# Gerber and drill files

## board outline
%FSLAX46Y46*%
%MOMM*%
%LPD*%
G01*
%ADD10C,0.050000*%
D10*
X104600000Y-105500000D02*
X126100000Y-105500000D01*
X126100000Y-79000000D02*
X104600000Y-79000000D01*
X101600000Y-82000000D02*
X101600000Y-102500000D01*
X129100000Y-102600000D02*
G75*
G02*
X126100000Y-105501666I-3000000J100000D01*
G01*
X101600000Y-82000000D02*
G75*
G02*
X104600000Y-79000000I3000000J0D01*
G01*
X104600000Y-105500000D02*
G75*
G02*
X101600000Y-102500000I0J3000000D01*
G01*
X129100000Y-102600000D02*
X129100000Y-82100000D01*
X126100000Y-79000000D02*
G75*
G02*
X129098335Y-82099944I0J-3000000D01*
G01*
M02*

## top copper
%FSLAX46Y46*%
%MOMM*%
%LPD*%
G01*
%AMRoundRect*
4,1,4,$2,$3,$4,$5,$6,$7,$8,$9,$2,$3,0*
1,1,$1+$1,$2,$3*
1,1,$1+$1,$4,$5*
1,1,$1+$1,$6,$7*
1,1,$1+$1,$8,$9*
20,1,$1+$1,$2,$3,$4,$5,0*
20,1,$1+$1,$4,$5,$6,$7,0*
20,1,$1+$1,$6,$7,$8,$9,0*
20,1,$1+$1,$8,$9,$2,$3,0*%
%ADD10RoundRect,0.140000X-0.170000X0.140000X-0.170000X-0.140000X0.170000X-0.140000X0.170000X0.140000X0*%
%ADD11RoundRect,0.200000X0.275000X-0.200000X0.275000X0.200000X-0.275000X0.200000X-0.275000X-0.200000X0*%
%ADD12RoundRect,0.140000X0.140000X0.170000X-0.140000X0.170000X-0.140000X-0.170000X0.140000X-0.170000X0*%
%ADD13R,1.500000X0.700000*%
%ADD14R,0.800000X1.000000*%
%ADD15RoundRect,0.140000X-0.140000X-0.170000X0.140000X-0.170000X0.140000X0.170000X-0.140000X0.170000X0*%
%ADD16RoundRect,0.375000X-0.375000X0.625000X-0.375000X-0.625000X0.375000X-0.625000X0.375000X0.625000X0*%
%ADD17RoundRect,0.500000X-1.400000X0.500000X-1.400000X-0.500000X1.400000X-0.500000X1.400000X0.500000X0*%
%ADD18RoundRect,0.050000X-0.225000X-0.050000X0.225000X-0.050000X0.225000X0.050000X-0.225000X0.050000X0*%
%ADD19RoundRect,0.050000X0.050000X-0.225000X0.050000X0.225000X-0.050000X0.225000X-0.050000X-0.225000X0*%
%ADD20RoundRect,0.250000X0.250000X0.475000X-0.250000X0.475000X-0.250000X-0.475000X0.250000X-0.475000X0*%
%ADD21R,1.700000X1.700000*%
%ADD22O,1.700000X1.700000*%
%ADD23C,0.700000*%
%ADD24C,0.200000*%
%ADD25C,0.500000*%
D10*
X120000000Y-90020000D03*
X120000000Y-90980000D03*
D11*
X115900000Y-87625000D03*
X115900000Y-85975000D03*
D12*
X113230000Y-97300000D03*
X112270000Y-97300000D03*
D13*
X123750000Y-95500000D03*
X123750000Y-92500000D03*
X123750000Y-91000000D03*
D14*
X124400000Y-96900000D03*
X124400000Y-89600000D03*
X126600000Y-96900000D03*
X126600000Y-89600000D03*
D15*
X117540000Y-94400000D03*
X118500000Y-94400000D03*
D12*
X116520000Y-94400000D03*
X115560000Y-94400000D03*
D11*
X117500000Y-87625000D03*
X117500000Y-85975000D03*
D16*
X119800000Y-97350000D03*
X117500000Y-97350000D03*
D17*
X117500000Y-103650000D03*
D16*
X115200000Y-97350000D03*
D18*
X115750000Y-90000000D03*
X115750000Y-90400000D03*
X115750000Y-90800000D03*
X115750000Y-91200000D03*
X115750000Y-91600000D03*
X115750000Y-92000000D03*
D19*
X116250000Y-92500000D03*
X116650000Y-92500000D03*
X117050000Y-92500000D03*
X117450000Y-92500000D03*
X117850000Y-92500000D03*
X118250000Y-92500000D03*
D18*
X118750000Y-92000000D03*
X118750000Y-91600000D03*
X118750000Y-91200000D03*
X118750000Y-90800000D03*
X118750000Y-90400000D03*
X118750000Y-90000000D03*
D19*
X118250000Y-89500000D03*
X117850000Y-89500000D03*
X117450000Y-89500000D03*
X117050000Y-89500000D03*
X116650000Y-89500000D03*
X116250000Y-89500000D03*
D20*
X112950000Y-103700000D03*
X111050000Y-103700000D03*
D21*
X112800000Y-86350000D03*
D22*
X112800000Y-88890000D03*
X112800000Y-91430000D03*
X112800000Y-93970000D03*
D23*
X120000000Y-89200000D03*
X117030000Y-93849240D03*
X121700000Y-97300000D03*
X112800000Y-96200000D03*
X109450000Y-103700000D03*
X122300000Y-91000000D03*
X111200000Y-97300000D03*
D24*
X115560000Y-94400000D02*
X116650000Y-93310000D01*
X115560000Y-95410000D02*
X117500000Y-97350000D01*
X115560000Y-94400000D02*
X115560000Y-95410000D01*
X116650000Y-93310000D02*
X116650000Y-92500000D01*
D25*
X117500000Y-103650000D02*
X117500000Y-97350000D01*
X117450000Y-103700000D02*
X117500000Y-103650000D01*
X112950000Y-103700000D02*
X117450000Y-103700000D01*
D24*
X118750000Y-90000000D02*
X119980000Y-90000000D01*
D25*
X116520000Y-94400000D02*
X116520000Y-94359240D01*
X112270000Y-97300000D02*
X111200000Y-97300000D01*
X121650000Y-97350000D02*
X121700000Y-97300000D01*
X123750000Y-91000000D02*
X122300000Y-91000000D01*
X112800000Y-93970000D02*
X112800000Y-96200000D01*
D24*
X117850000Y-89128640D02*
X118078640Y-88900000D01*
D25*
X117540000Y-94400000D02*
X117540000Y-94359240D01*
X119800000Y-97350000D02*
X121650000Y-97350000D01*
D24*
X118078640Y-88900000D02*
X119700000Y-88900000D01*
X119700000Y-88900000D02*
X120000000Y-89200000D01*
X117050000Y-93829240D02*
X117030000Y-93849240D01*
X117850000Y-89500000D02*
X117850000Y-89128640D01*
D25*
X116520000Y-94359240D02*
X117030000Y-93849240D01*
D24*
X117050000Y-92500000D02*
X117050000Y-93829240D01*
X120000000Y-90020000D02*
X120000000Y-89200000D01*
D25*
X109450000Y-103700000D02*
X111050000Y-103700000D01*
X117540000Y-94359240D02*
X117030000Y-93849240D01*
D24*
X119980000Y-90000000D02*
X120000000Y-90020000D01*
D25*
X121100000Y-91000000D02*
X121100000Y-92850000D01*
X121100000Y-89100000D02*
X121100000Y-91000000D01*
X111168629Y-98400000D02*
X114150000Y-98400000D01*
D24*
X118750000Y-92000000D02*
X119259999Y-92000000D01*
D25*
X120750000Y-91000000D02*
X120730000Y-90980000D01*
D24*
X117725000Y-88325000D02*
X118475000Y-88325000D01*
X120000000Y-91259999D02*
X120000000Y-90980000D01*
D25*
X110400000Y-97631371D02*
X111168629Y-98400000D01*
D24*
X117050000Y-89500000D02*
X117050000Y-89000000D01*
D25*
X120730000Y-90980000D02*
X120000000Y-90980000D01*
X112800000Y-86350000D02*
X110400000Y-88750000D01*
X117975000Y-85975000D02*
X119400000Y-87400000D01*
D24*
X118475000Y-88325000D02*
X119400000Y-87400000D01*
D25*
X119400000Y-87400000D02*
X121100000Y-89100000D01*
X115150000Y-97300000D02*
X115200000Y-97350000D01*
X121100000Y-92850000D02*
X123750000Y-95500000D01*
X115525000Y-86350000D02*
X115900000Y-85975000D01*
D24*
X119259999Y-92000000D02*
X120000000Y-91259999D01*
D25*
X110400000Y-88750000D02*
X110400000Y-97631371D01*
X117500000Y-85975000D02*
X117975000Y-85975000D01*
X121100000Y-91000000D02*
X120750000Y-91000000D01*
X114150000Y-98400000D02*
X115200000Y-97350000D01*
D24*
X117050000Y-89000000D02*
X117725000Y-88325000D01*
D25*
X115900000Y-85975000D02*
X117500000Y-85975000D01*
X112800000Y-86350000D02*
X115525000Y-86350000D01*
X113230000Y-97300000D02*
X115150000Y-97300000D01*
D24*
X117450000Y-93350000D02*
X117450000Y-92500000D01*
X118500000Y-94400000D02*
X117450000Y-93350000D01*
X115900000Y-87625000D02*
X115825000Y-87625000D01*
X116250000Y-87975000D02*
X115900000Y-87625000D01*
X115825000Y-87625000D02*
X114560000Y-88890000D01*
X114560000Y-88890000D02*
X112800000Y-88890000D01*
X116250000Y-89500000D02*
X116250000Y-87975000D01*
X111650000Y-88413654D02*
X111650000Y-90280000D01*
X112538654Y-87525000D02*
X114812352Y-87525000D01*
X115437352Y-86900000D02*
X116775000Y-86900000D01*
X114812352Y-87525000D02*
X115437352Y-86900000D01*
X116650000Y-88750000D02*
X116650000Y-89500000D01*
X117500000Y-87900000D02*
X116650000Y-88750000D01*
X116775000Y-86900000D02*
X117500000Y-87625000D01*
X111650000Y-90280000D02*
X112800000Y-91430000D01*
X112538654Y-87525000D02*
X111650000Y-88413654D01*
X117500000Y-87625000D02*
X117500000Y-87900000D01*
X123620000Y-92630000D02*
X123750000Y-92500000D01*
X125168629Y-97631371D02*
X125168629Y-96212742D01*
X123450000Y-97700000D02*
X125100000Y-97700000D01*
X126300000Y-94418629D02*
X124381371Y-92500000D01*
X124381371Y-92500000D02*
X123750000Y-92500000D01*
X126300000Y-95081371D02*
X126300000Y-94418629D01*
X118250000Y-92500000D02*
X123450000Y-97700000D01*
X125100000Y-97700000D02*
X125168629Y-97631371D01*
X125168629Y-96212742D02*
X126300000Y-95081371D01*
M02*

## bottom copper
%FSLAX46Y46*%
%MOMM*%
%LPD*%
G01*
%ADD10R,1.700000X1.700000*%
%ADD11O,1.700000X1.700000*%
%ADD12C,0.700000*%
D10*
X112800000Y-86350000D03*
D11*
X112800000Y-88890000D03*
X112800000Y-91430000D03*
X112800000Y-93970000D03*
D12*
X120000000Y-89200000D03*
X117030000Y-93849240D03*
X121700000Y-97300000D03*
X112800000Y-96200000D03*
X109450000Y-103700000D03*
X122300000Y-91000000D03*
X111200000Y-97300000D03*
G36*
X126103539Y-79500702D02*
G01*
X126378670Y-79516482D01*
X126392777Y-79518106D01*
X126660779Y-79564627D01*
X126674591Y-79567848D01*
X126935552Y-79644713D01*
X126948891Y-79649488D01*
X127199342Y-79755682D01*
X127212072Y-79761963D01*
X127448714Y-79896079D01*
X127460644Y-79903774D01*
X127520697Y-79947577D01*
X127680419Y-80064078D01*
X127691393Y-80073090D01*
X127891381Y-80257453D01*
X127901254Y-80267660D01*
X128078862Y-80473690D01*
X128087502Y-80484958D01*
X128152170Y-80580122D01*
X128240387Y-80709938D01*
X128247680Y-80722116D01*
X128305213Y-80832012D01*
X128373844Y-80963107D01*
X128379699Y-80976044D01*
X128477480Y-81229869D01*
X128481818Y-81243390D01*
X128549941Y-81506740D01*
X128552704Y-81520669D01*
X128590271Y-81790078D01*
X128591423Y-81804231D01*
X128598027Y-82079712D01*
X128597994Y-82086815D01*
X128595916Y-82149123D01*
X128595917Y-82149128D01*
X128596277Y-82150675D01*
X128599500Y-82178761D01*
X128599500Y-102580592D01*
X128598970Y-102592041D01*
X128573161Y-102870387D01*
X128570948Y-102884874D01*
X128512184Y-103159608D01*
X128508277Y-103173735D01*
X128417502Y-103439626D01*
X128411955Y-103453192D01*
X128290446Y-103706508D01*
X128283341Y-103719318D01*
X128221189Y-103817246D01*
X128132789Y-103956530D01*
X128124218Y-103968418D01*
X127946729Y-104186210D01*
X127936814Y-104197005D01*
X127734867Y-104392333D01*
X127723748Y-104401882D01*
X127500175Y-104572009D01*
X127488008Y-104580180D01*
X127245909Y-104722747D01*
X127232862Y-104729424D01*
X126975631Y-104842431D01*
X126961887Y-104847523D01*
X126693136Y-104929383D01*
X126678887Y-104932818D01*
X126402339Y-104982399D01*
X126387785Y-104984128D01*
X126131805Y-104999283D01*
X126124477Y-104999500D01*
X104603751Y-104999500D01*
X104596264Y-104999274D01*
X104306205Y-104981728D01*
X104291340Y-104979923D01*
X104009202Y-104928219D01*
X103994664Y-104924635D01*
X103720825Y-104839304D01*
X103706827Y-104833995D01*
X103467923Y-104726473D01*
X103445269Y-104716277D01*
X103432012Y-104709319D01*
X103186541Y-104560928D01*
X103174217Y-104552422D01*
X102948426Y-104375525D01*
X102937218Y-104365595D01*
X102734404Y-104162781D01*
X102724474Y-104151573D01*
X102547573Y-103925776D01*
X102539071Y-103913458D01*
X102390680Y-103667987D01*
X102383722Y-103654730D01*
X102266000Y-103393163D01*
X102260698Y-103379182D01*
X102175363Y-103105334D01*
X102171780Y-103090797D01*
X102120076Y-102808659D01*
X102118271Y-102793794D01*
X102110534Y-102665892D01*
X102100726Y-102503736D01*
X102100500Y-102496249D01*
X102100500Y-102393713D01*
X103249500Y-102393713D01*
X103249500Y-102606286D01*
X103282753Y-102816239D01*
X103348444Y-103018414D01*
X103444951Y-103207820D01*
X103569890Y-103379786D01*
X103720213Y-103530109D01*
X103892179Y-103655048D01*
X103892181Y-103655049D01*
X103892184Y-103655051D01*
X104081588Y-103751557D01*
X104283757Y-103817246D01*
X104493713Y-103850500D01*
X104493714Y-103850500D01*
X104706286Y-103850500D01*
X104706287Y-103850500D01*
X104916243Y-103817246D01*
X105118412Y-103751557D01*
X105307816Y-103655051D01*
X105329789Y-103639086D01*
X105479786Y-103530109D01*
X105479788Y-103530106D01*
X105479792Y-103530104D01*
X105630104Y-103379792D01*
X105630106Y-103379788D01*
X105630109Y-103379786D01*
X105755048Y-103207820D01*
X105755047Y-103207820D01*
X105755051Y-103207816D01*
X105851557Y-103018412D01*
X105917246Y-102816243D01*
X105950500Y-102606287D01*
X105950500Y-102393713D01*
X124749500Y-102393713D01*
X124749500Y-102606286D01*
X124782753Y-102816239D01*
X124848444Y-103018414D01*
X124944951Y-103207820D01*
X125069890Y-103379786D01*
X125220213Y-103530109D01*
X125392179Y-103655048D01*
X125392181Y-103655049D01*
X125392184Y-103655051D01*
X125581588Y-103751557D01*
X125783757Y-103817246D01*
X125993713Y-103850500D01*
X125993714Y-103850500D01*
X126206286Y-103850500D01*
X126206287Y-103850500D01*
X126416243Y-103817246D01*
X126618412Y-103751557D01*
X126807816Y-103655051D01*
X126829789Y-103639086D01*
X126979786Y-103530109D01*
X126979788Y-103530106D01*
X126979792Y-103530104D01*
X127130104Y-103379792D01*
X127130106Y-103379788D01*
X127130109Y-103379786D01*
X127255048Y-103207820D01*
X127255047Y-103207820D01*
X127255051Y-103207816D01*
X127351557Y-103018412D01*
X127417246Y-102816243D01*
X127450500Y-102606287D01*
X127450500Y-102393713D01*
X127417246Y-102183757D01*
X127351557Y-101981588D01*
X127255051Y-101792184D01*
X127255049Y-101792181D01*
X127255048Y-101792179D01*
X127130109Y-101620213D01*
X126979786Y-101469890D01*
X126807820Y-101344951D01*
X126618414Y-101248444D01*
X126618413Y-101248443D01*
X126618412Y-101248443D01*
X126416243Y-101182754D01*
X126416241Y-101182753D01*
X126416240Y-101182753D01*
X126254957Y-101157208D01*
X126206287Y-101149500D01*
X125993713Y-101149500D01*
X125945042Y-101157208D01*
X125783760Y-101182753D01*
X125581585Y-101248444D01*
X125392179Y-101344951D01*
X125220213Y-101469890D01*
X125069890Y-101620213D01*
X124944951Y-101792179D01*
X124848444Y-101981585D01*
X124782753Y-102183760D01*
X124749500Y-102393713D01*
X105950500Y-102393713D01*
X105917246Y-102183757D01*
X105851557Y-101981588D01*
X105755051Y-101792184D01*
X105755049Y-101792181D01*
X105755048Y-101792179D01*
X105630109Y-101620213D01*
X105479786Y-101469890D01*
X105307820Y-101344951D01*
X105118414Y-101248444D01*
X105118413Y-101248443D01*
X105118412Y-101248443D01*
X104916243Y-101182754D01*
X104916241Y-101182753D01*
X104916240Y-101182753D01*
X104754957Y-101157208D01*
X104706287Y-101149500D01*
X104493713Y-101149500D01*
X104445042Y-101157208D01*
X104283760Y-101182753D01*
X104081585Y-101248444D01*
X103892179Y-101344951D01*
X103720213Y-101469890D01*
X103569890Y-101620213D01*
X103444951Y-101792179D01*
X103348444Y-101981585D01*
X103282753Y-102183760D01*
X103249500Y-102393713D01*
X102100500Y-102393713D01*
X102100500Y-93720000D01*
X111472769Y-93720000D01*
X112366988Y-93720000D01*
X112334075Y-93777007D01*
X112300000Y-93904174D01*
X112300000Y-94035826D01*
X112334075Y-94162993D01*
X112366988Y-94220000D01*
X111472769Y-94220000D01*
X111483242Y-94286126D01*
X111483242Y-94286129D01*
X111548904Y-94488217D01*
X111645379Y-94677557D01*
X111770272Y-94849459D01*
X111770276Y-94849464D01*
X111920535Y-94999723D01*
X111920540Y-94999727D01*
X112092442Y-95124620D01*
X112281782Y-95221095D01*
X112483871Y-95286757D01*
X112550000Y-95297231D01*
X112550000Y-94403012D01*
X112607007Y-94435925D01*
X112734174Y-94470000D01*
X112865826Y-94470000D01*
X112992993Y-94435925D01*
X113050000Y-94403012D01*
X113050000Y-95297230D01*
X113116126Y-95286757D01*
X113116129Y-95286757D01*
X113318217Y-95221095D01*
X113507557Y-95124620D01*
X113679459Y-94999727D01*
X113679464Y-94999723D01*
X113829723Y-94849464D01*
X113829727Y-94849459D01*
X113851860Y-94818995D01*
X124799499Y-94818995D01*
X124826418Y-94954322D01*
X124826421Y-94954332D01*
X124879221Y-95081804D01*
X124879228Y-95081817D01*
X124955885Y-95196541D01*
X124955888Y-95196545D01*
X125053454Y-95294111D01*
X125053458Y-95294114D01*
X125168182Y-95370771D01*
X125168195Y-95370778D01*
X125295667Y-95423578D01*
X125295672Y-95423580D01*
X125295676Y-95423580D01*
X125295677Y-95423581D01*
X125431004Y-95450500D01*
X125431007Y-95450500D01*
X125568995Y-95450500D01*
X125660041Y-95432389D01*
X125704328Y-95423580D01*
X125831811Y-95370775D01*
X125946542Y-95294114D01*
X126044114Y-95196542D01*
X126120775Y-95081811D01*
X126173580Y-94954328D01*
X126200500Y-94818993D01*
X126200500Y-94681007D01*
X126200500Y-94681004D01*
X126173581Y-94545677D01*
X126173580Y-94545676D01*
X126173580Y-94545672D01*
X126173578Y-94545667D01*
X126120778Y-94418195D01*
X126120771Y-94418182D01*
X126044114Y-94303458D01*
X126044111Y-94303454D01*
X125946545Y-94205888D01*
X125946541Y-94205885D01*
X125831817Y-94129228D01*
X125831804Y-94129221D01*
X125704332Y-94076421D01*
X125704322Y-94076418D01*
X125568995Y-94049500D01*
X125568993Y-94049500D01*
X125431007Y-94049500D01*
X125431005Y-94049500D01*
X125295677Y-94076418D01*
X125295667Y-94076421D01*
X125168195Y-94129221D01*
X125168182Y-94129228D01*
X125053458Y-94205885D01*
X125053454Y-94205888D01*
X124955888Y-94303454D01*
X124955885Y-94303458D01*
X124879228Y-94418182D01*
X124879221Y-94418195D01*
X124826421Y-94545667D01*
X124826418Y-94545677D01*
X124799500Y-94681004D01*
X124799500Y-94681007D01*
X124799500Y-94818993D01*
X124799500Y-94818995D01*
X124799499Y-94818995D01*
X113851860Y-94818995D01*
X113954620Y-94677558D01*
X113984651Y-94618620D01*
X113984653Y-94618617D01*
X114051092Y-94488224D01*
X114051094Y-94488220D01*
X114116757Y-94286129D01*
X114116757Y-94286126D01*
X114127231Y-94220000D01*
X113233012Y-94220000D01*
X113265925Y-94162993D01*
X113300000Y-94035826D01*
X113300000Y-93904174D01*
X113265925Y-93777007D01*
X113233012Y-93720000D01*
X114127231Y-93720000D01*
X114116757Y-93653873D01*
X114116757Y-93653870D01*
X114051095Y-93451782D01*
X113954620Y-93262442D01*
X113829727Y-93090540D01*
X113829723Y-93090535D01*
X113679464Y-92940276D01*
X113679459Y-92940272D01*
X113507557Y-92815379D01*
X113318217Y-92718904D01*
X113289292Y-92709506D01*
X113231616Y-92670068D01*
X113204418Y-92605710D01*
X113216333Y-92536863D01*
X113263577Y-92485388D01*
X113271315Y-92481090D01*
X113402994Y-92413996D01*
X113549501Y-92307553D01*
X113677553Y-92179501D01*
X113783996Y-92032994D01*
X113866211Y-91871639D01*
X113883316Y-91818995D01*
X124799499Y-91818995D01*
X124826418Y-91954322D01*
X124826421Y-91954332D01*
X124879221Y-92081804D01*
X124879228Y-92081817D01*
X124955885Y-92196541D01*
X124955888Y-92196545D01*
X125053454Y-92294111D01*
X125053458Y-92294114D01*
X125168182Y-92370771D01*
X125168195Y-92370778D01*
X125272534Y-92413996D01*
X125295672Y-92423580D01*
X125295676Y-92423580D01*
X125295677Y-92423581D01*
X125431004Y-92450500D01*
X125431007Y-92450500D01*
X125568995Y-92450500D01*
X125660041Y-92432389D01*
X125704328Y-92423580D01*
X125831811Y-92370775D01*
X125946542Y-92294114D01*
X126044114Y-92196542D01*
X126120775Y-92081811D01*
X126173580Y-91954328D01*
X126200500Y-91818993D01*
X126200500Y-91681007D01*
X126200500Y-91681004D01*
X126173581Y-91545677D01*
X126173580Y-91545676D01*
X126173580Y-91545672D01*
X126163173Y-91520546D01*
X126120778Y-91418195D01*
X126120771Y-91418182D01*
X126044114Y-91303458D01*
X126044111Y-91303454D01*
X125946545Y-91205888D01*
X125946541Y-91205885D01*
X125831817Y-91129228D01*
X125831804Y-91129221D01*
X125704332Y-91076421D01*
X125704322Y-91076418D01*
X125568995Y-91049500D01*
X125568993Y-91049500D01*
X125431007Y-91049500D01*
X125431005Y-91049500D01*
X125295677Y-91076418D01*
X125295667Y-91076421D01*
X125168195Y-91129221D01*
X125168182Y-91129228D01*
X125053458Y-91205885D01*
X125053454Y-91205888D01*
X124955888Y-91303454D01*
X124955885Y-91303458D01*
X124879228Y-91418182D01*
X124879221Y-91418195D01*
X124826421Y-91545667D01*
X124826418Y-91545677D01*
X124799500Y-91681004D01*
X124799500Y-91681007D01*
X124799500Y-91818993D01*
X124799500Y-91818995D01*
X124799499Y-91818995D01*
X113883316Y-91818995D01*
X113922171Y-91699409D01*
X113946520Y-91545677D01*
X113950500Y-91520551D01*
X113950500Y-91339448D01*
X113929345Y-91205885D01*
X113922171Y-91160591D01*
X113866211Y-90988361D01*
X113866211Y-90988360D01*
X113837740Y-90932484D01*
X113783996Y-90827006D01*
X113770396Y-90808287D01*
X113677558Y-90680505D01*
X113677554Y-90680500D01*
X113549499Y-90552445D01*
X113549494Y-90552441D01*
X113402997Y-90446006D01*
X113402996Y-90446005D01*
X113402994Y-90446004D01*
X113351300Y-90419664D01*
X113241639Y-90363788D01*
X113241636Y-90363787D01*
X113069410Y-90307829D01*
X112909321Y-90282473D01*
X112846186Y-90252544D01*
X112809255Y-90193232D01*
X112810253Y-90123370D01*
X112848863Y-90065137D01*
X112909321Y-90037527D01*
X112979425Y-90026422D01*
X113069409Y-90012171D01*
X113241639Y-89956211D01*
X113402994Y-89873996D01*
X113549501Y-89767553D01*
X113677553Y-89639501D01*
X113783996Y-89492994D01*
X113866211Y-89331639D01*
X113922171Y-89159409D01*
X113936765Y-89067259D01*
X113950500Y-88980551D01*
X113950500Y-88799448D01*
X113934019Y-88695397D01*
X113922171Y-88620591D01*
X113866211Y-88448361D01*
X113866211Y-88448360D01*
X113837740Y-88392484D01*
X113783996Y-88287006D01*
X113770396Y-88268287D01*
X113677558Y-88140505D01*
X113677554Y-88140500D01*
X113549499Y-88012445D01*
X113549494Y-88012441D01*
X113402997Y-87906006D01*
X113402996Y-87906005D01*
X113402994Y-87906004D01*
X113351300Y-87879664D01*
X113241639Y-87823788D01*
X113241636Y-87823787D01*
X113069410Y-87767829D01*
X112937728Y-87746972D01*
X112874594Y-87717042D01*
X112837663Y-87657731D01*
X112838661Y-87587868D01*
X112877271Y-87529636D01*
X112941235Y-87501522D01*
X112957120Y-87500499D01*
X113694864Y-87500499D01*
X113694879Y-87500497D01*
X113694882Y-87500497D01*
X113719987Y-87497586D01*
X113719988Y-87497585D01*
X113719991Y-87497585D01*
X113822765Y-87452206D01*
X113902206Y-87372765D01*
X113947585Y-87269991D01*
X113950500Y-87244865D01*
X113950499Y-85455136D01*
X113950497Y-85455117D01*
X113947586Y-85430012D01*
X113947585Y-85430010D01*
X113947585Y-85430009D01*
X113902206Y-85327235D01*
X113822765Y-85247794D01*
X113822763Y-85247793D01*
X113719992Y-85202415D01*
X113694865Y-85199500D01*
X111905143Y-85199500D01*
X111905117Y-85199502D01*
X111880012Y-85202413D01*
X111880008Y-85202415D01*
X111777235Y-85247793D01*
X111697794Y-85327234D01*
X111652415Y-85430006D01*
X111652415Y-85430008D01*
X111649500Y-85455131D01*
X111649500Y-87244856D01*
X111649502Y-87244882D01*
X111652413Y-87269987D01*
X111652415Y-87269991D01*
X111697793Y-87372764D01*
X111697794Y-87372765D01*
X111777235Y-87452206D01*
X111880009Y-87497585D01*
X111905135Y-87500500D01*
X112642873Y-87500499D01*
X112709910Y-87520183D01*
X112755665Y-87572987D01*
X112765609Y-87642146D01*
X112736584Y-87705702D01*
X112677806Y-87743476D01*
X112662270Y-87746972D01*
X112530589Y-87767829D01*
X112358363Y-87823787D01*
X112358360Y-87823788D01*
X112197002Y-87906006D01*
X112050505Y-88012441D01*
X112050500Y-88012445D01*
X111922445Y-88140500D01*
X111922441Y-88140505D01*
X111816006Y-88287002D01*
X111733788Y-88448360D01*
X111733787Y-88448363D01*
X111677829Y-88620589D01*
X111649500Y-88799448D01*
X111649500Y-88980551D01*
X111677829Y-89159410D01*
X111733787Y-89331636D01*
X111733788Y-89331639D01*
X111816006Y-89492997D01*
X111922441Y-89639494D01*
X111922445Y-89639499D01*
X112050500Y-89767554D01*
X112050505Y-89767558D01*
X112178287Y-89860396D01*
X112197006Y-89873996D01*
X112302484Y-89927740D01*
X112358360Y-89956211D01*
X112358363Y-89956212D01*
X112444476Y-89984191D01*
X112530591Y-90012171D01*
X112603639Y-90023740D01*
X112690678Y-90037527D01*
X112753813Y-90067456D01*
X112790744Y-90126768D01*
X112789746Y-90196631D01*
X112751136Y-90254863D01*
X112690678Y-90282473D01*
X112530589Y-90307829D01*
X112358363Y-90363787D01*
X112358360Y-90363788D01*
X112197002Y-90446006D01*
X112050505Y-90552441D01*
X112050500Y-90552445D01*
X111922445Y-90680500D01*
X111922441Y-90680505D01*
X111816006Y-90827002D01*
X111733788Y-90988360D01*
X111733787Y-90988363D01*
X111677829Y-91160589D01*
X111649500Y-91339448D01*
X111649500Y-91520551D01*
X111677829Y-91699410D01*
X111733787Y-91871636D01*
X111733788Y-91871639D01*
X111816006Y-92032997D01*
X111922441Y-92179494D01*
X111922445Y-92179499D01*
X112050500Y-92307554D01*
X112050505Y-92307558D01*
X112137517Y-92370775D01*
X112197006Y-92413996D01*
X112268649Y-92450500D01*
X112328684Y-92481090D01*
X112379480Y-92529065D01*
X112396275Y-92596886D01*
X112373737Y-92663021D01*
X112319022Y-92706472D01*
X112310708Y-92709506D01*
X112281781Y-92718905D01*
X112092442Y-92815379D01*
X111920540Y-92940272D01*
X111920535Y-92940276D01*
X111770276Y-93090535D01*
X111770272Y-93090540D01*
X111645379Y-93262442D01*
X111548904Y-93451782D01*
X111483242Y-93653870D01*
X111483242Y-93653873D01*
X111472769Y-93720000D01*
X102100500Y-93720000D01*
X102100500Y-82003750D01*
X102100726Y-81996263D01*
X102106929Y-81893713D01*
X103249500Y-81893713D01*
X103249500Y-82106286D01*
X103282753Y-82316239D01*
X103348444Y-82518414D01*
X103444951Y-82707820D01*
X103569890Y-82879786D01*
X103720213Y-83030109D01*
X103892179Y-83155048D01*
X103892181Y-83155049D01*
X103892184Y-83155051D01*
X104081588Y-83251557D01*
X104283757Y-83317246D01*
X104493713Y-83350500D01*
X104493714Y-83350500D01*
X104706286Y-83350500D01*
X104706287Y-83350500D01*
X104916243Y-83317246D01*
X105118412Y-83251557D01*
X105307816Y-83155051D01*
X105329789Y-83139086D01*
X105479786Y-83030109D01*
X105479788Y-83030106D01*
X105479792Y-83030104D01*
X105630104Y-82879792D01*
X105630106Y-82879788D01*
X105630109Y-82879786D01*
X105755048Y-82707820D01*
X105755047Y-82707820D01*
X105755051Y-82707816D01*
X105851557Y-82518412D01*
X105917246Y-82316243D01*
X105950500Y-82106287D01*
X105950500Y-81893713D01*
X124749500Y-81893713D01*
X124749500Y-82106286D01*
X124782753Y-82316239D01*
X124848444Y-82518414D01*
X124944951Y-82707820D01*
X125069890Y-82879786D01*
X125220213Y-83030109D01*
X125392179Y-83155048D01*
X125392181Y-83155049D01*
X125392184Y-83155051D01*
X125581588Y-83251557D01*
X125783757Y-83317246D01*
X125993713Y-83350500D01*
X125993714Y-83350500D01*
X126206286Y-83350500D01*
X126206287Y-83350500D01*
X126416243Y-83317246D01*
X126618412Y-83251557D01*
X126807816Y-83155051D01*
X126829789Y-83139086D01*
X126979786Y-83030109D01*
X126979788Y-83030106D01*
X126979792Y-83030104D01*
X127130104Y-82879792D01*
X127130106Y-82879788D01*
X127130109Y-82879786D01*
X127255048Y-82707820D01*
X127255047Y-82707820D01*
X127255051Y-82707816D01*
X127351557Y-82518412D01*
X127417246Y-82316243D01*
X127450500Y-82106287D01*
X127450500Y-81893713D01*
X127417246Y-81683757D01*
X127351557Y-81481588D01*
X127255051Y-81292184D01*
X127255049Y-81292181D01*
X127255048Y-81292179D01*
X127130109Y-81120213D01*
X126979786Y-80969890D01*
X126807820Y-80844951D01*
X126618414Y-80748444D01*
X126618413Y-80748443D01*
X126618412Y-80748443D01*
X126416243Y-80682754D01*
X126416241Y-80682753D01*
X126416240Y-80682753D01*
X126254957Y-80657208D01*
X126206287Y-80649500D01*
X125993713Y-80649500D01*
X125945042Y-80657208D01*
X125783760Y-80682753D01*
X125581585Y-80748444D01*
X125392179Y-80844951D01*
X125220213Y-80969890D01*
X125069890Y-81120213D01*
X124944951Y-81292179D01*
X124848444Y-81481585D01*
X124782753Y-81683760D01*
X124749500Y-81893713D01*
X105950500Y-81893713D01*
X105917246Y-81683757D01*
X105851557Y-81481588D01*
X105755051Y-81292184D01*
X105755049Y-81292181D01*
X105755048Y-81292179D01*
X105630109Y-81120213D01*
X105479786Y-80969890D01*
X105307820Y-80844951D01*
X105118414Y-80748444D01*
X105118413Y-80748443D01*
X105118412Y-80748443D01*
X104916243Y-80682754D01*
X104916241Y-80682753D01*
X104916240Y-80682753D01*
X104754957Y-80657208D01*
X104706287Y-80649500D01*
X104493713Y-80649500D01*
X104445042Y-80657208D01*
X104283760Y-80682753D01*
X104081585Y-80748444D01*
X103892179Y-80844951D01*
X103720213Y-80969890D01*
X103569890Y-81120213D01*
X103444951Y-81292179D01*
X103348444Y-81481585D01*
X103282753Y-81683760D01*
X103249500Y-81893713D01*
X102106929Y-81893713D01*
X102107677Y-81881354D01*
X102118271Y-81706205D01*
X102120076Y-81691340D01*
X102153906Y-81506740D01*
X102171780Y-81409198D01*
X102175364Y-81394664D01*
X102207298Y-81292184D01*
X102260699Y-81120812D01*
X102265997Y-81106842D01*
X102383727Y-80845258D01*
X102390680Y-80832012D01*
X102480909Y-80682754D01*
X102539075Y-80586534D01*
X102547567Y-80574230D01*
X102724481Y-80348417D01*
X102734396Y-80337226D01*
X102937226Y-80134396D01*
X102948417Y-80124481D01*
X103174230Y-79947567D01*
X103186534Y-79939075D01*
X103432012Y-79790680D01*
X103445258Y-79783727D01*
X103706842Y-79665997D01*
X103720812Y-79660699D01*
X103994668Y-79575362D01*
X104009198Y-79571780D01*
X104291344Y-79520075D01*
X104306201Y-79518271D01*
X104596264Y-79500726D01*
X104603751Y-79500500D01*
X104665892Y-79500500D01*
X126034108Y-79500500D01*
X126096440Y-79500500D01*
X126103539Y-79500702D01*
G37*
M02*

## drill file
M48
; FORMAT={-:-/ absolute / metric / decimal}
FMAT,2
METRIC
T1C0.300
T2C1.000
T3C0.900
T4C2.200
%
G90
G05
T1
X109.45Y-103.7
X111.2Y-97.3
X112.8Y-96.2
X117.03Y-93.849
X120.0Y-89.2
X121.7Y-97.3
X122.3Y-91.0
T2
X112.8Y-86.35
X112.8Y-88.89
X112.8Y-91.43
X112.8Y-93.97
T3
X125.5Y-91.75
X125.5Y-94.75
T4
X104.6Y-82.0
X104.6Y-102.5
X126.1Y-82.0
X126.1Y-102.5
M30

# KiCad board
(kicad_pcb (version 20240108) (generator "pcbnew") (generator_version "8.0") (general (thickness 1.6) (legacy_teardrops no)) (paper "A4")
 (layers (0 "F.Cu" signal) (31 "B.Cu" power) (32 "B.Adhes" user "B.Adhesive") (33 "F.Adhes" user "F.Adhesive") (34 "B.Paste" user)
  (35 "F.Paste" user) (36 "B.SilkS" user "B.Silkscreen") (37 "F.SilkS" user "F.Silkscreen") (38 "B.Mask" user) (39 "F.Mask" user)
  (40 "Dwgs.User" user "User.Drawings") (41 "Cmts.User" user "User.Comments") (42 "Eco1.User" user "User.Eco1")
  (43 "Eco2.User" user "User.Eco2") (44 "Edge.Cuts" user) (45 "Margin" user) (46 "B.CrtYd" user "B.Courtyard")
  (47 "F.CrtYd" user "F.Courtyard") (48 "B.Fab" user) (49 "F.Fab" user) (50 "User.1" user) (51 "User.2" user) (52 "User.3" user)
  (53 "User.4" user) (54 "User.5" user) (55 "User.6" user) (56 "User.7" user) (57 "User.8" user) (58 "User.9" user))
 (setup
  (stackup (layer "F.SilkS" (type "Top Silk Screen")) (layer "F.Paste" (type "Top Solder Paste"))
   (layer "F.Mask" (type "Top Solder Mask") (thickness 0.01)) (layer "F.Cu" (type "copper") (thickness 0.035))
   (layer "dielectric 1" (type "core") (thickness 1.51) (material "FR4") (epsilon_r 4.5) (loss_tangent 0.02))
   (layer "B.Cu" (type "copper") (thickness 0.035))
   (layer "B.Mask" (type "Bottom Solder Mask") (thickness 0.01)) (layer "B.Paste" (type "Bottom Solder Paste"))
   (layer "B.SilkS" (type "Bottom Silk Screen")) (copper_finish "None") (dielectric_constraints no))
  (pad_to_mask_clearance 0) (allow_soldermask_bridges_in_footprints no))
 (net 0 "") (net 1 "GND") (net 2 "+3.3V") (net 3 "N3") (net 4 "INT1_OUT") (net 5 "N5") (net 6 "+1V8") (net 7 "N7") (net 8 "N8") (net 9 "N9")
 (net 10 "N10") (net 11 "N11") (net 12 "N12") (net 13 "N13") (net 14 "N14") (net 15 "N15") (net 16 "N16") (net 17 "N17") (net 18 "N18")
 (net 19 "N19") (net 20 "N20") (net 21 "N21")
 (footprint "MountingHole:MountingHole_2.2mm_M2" (layer "F.Cu") (at 126.1 102.5)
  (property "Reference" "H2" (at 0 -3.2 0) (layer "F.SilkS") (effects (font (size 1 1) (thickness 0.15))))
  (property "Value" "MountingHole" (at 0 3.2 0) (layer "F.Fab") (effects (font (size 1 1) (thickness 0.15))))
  (pad "" np_thru_hole circle (at 0 0) (size 2.2 2.2) (drill 2.2) (layers "*.Cu" "*.Mask")))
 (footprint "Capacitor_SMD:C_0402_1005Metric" (layer "F.Cu") (at 120 90.5 -90)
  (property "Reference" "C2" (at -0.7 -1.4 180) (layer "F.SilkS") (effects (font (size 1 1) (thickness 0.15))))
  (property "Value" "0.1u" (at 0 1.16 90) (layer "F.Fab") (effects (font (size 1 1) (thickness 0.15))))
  (pad "1" smd roundrect (at -0.48 0 270) (size 0.56 0.62) (layers "F.Cu" "F.Paste" "F.Mask") (roundrect_rratio 0.25) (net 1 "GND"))
  (pad "2" smd roundrect (at 0.48 0 270) (size 0.56 0.62) (layers "F.Cu" "F.Paste" "F.Mask") (roundrect_rratio 0.25) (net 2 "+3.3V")))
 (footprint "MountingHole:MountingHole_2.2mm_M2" (layer "F.Cu") (at 104.6 102.5)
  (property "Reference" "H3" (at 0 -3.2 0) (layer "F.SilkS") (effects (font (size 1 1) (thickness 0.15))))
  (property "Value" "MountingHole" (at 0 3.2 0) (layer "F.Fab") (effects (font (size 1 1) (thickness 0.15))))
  (pad "" np_thru_hole circle (at 0 0) (size 2.2 2.2) (drill 2.2) (layers "*.Cu" "*.Mask")))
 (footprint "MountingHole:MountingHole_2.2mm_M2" (layer "F.Cu") (at 104.6 82)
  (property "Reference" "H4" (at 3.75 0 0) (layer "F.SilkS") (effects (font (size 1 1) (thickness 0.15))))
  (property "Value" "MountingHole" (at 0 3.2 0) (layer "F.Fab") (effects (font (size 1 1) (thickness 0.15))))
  (pad "" np_thru_hole circle (at 0 0) (size 2.2 2.2) (drill 2.2) (layers "*.Cu" "*.Mask")))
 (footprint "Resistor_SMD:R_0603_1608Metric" (layer "F.Cu") (at 115.9 86.8 90)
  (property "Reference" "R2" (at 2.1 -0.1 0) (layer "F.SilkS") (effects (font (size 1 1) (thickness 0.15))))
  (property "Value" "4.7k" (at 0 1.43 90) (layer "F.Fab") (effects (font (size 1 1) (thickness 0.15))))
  (pad "1" smd roundrect (at -0.825 0 90) (size 0.8 0.95) (layers "F.Cu" "F.Paste" "F.Mask") (roundrect_rratio 0.25) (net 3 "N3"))
  (pad "2" smd roundrect (at 0.825 0 90) (size 0.8 0.95) (layers "F.Cu" "F.Paste" "F.Mask") (roundrect_rratio 0.25) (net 2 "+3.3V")))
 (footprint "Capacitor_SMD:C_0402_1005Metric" (layer "F.Cu") (at 112.75 97.3 180)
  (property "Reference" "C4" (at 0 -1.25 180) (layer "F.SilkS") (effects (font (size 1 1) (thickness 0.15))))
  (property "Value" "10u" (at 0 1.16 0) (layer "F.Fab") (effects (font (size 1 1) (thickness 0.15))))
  (pad "1" smd roundrect (at -0.48 0 180) (size 0.56 0.62) (layers "F.Cu" "F.Paste" "F.Mask") (roundrect_rratio 0.25) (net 2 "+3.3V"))
  (pad "2" smd roundrect (at 0.48 0 180) (size 0.56 0.62) (layers "F.Cu" "F.Paste" "F.Mask") (roundrect_rratio 0.25) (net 1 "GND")))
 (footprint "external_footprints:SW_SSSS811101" (layer "F.Cu") (at 125.5 93.25 90)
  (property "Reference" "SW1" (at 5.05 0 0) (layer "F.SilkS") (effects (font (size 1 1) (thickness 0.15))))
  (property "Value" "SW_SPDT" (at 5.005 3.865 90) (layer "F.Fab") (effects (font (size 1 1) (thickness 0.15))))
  (pad "" np_thru_hole circle (at -1.5 0 90) (size 0.9 0.9) (drill 0.9) (layers "*.Cu" "*.Mask"))
  (pad "" np_thru_hole circle (at 1.5 0 90) (size 0.9 0.9) (drill 0.9) (layers "*.Cu" "*.Mask"))
  (pad "1" smd rect (at -2.25 -1.75 90) (size 0.7 1.5) (layers "F.Cu" "F.Paste" "F.Mask") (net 2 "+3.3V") (solder_mask_margin 0.102))
  (pad "2" smd rect (at 0.75 -1.75 90) (size 0.7 1.5) (layers "F.Cu" "F.Paste" "F.Mask") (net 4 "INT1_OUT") (solder_mask_margin 0.102))
  (pad "3" smd rect (at 2.25 -1.75 90) (size 0.7 1.5) (layers "F.Cu" "F.Paste" "F.Mask") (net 1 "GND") (solder_mask_margin 0.102))
  (pad "SH1" smd rect (at -3.65 -1.1 90) (size 1 0.8) (layers "F.Cu" "F.Paste" "F.Mask") (solder_mask_margin 0.102))
  (pad "SH2" smd rect (at 3.65 -1.1 90) (size 1 0.8) (layers "F.Cu" "F.Paste" "F.Mask") (solder_mask_margin 0.102))
  (pad "SH3" smd rect (at -3.65 1.1 90) (size 1 0.8) (layers "F.Cu" "F.Paste" "F.Mask") (solder_mask_margin 0.102))
  (pad "SH4" smd rect (at 3.65 1.1 90) (size 1 0.8) (layers "F.Cu" "F.Paste" "F.Mask") (solder_mask_margin 0.102)))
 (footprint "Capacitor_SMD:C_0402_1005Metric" (layer "F.Cu") (at 118.02 94.4)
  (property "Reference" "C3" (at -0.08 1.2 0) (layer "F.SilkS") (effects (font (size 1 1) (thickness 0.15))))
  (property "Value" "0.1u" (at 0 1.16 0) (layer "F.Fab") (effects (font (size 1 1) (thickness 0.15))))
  (pad "1" smd roundrect (at -0.48 0) (size 0.56 0.62) (layers "F.Cu" "F.Paste" "F.Mask") (roundrect_rratio 0.25) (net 1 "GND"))
  (pad "2" smd roundrect (at 0.48 0) (size 0.56 0.62) (layers "F.Cu" "F.Paste" "F.Mask") (roundrect_rratio 0.25) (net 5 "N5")))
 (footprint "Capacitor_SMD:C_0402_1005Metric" (layer "F.Cu") (at 116.04 94.4 180)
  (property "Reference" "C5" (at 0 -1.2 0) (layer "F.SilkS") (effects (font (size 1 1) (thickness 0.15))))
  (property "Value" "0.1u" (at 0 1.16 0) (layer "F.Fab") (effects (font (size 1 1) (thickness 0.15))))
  (pad "1" smd roundrect (at -0.48 0 180) (size 0.56 0.62) (layers "F.Cu" "F.Paste" "F.Mask") (roundrect_rratio 0.25) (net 1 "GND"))
  (pad "2" smd roundrect (at 0.48 0 180) (size 0.56 0.62) (layers "F.Cu" "F.Paste" "F.Mask") (roundrect_rratio 0.25) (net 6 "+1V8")))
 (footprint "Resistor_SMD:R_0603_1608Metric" (layer "F.Cu") (at 117.5 86.8 90)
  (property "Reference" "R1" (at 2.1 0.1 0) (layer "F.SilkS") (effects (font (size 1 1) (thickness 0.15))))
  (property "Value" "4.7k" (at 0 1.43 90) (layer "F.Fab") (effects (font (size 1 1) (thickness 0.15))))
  (pad "1" smd roundrect (at -0.825 0 90) (size 0.8 0.95) (layers "F.Cu" "F.Paste" "F.Mask") (roundrect_rratio 0.25) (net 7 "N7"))
  (pad "2" smd roundrect (at 0.825 0 90) (size 0.8 0.95) (layers "F.Cu" "F.Paste" "F.Mask") (roundrect_rratio 0.25) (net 2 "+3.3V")))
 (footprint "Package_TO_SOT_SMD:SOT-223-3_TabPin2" (layer "F.Cu") (at 117.5 100.5 -90)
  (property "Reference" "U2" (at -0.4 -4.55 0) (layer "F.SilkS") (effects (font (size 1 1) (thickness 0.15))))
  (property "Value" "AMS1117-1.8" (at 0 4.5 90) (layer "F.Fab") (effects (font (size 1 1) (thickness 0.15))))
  (pad "1" smd roundrect (at -3.15 -2.3 270) (size 2 1.5) (layers "F.Cu" "F.Paste" "F.Mask") (roundrect_rratio 0.25) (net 1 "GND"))
  (pad "2" smd roundrect (at -3.15 0 270) (size 2 1.5) (layers "F.Cu" "F.Paste" "F.Mask") (roundrect_rratio 0.25) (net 6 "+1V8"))
  (pad "2" smd roundrect (at 3.15 0 270) (size 2 3.8) (layers "F.Cu" "F.Paste" "F.Mask") (roundrect_rratio 0.25) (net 6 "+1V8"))
  (pad "3" smd roundrect (at -3.15 2.3 270) (size 2 1.5) (layers "F.Cu" "F.Paste" "F.Mask") (roundrect_rratio 0.25) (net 2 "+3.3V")))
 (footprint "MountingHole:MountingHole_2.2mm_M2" (layer "F.Cu") (at 126.1 82)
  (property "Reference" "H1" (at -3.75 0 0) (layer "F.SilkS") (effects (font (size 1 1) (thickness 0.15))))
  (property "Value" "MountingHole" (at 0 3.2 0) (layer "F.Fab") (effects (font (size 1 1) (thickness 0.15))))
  (pad "" np_thru_hole circle (at 0 0) (size 2.2 2.2) (drill 2.2) (layers "*.Cu" "*.Mask")))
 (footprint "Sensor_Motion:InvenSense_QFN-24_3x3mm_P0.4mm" (layer "F.Cu") (at 117.25 91)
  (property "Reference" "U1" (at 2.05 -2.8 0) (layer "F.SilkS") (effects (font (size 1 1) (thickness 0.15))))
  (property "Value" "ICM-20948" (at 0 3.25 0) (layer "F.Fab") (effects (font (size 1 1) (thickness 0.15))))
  (pad "1" smd roundrect (at -1.5 -1) (size 0.55 0.2) (layers "F.Cu" "F.Paste" "F.Mask") (roundrect_rratio 0.25) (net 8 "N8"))
  (pad "2" smd roundrect (at -1.5 -0.6) (size 0.55 0.2) (layers "F.Cu" "F.Paste" "F.Mask") (roundrect_rratio 0.25) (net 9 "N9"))
  (pad "3" smd roundrect (at -1.5 -0.2) (size 0.55 0.2) (layers "F.Cu" "F.Paste" "F.Mask") (roundrect_rratio 0.25) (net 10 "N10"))
  (pad "4" smd roundrect (at -1.5 0.2) (size 0.55 0.2) (layers "F.Cu" "F.Paste" "F.Mask") (roundrect_rratio 0.25) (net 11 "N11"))
  (pad "5" smd roundrect (at -1.5 0.6) (size 0.55 0.2) (layers "F.Cu" "F.Paste" "F.Mask") (roundrect_rratio 0.25) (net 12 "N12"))
  (pad "6" smd roundrect (at -1.5 1) (size 0.55 0.2) (layers "F.Cu" "F.Paste" "F.Mask") (roundrect_rratio 0.25) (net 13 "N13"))
  (pad "7" smd roundrect (at -1 1.5 90) (size 0.55 0.2) (layers "F.Cu" "F.Paste" "F.Mask") (roundrect_rratio 0.25) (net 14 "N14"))
  (pad "8" smd roundrect (at -0.6 1.5 90) (size 0.55 0.2) (layers "F.Cu" "F.Paste" "F.Mask") (roundrect_rratio 0.25) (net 6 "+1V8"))
  (pad "9" smd roundrect (at -0.2 1.5 90) (size 0.55 0.2) (layers "F.Cu" "F.Paste" "F.Mask") (roundrect_rratio 0.25) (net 1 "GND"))
  (pad "10" smd roundrect (at 0.2 1.5 90) (size 0.55 0.2) (layers "F.Cu" "F.Paste" "F.Mask") (roundrect_rratio 0.25) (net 5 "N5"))
  (pad "11" smd roundrect (at 0.6 1.5 90) (size 0.55 0.2) (layers "F.Cu" "F.Paste" "F.Mask") (roundrect_rratio 0.25) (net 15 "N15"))
  (pad "12" smd roundrect (at 1 1.5 90) (size 0.55 0.2) (layers "F.Cu" "F.Paste" "F.Mask") (roundrect_rratio 0.25) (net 4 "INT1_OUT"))
  (pad "13" smd roundrect (at 1.5 1) (size 0.55 0.2) (layers "F.Cu" "F.Paste" "F.Mask") (roundrect_rratio 0.25) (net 2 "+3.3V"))
  (pad "14" smd roundrect (at 1.5 0.6) (size 0.55 0.2) (layers "F.Cu" "F.Paste" "F.Mask") (roundrect_rratio 0.25) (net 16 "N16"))
  (pad "15" smd roundrect (at 1.5 0.2) (size 0.55 0.2) (layers "F.Cu" "F.Paste" "F.Mask") (roundrect_rratio 0.25) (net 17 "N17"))
  (pad "16" smd roundrect (at 1.5 -0.2) (size 0.55 0.2) (layers "F.Cu" "F.Paste" "F.Mask") (roundrect_rratio 0.25) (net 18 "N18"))
  (pad "17" smd roundrect (at 1.5 -0.6) (size 0.55 0.2) (layers "F.Cu" "F.Paste" "F.Mask") (roundrect_rratio 0.25) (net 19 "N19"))
  (pad "18" smd roundrect (at 1.5 -1) (size 0.55 0.2) (layers "F.Cu" "F.Paste" "F.Mask") (roundrect_rratio 0.25) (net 1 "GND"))
  (pad "19" smd roundrect (at 1 -1.5 90) (size 0.55 0.2) (layers "F.Cu" "F.Paste" "F.Mask") (roundrect_rratio 0.25) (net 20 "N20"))
  (pad "20" smd roundrect (at 0.6 -1.5 90) (size 0.55 0.2) (layers "F.Cu" "F.Paste" "F.Mask") (roundrect_rratio 0.25) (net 1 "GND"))
  (pad "21" smd roundrect (at 0.2 -1.5 90) (size 0.55 0.2) (layers "F.Cu" "F.Paste" "F.Mask") (roundrect_rratio 0.25) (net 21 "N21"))
  (pad "22" smd roundrect (at -0.2 -1.5 90) (size 0.55 0.2) (layers "F.Cu" "F.Paste" "F.Mask") (roundrect_rratio 0.25) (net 2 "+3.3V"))
  (pad "23" smd roundrect (at -0.6 -1.5 90) (size 0.55 0.2) (layers "F.Cu" "F.Paste" "F.Mask") (roundrect_rratio 0.25) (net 7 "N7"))
  (pad "24" smd roundrect (at -1 -1.5 90) (size 0.55 0.2) (layers "F.Cu" "F.Paste" "F.Mask") (roundrect_rratio 0.25) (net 3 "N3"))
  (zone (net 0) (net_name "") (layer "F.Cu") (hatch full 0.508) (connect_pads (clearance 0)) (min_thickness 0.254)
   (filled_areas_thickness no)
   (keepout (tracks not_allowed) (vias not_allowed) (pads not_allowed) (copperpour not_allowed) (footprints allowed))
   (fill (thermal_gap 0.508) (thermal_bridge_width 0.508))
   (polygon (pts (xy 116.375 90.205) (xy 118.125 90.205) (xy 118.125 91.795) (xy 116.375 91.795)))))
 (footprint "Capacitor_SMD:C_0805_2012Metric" (layer "F.Cu") (at 112 103.7 180)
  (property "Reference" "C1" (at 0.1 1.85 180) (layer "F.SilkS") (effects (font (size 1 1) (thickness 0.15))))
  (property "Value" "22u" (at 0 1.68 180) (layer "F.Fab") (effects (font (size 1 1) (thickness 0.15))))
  (pad "1" smd roundrect (at -0.95 0 180) (size 1 1.45) (layers "F.Cu" "F.Paste" "F.Mask") (roundrect_rratio 0.25) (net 6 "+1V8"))
  (pad "2" smd roundrect (at 0.95 0 180) (size 1 1.45) (layers "F.Cu" "F.Paste" "F.Mask") (roundrect_rratio 0.25) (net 1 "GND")))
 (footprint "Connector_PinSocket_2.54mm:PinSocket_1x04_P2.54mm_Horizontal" (layer "F.Cu") (at 112.8 86.35)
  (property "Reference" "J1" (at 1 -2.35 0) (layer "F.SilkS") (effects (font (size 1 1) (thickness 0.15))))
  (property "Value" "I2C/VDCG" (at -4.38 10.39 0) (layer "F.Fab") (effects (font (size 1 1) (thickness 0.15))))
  (pad "1" thru_hole rect (at 0 0) (size 1.7 1.7) (drill 1) (layers "*.Cu" "*.Mask") (remove_unused_layers no) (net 2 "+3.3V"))
  (pad "2" thru_hole oval (at 0 2.54) (size 1.7 1.7) (drill 1) (layers "*.Cu" "*.Mask") (remove_unused_layers no) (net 3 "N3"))
  (pad "3" thru_hole oval (at 0 5.08) (size 1.7 1.7) (drill 1) (layers "*.Cu" "*.Mask") (remove_unused_layers no) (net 7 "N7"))
  (pad "4" thru_hole oval (at 0 7.62) (size 1.7 1.7) (drill 1) (layers "*.Cu" "*.Mask") (remove_unused_layers no) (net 1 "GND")))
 (gr_line (start 104.6 105.5) (end 126.1 105.5) (stroke (width 0.05) (type default)) (layer "Edge.Cuts"))
 (gr_line (start 126.1 79) (end 104.6 79) (stroke (width 0.05) (type default)) (layer "Edge.Cuts"))
 (gr_line (start 101.6 82) (end 101.6 102.5) (stroke (width 0.05) (type default)) (layer "Edge.Cuts"))
 (gr_arc (start 129.1 102.6) (mid 128.186844 104.657564) (end 126.1 105.501666) (stroke (width 0.05) (type default)) (layer "Edge.Cuts"))
 (gr_arc (start 101.6 82) (mid 102.47868 79.87868) (end 104.6 79) (stroke (width 0.05) (type default)) (layer "Edge.Cuts"))
 (gr_arc (start 104.6 105.5) (mid 102.47868 104.62132) (end 101.6 102.5) (stroke (width 0.05) (type default)) (layer "Edge.Cuts"))
 (gr_line (start 129.1 102.6) (end 129.1 82.1) (stroke (width 0.05) (type default)) (layer "Edge.Cuts"))
 (gr_arc (start 126.1 79) (mid 128.256366 79.914314) (end 129.098335 82.099944) (stroke (width 0.05) (type default)) (layer "Edge.Cuts"))
 (segment (start 115.56 94.4) (end 116.65 93.31) (width 0.2) (layer "F.Cu") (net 6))
 (segment (start 115.56 95.41) (end 117.5 97.35) (width 0.2) (layer "F.Cu") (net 6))
 (segment (start 115.56 94.4) (end 115.56 95.41) (width 0.2) (layer "F.Cu") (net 6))
 (segment (start 116.65 93.31) (end 116.65 92.5) (width 0.2) (layer "F.Cu") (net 6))
 (segment (start 117.5 103.65) (end 117.5 97.35) (width 0.5) (layer "F.Cu") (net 6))
 (segment (start 117.45 103.7) (end 117.5 103.65) (width 0.5) (layer "F.Cu") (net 6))
 (segment (start 112.95 103.7) (end 117.45 103.7) (width 0.5) (layer "F.Cu") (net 6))
 (segment (start 118.75 90) (end 119.98 90) (width 0.2) (layer "F.Cu") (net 1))
 (segment (start 116.52 94.4) (end 116.52 94.35924) (width 0.5) (layer "F.Cu") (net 1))
 (segment (start 112.27 97.3) (end 111.2 97.3) (width 0.5) (layer "F.Cu") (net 1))
 (segment (start 121.65 97.35) (end 121.7 97.3) (width 0.5) (layer "F.Cu") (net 1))
 (segment (start 123.75 91) (end 122.3 91) (width 0.5) (layer "F.Cu") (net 1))
 (segment (start 112.8 93.97) (end 112.8 96.2) (width 0.5) (layer "F.Cu") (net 1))
 (segment (start 117.85 89.12864) (end 118.07864 88.9) (width 0.2) (layer "F.Cu") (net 1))
 (segment (start 117.54 94.4) (end 117.54 94.35924) (width 0.5) (layer "F.Cu") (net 1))
 (segment (start 119.8 97.35) (end 121.65 97.35) (width 0.5) (layer "F.Cu") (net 1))
 (segment (start 118.07864 88.9) (end 119.7 88.9) (width 0.2) (layer "F.Cu") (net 1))
 (segment (start 119.7 88.9) (end 120 89.2) (width 0.2) (layer "F.Cu") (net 1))
 (segment (start 117.05 93.82924) (end 117.03 93.84924) (width 0.2) (layer "F.Cu") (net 1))
 (segment (start 117.85 89.5) (end 117.85 89.12864) (width 0.2) (layer "F.Cu") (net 1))
 (segment (start 116.52 94.35924) (end 117.03 93.84924) (width 0.5) (layer "F.Cu") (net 1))
 (segment (start 117.05 92.5) (end 117.05 93.82924) (width 0.2) (layer "F.Cu") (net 1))
 (segment (start 120 90.02) (end 120 89.2) (width 0.2) (layer "F.Cu") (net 1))
 (segment (start 109.45 103.7) (end 111.05 103.7) (width 0.5) (layer "F.Cu") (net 1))
 (segment (start 117.54 94.35924) (end 117.03 93.84924) (width 0.5) (layer "F.Cu") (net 1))
 (segment (start 119.98 90) (end 120 90.02) (width 0.2) (layer "F.Cu") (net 1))
 (via (at 120 89.2) (size 0.7) (drill 0.3) (layers "F.Cu" "B.Cu") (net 1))
 (via (at 117.03 93.84924) (size 0.7) (drill 0.3) (layers "F.Cu" "B.Cu") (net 1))
 (via (at 121.7 97.3) (size 0.7) (drill 0.3) (layers "F.Cu" "B.Cu") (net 1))
 (via (at 112.8 96.2) (size 0.7) (drill 0.3) (layers "F.Cu" "B.Cu") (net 1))
 (via (at 109.45 103.7) (size 0.7) (drill 0.3) (layers "F.Cu" "B.Cu") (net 1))
 (via (at 122.3 91) (size 0.7) (drill 0.3) (layers "F.Cu" "B.Cu") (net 1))
 (via (at 111.2 97.3) (size 0.7) (drill 0.3) (layers "F.Cu" "B.Cu") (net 1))
 (segment (start 121.1 91) (end 121.1 92.85) (width 0.5) (layer "F.Cu") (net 2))
 (segment (start 121.1 89.1) (end 121.1 91) (width 0.5) (layer "F.Cu") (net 2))
 (segment (start 111.168629 98.4) (end 114.15 98.4) (width 0.5) (layer "F.Cu") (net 2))
 (segment (start 118.75 92) (end 119.259999 92) (width 0.2) (layer "F.Cu") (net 2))
 (segment (start 120.75 91) (end 120.73 90.98) (width 0.5) (layer "F.Cu") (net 2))
 (segment (start 117.725 88.325) (end 118.475 88.325) (width 0.2) (layer "F.Cu") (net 2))
 (segment (start 120 91.259999) (end 120 90.98) (width 0.2) (layer "F.Cu") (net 2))
 (segment (start 110.4 97.631371) (end 111.168629 98.4) (width 0.5) (layer "F.Cu") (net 2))
 (segment (start 117.05 89.5) (end 117.05 89) (width 0.2) (layer "F.Cu") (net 2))
 (segment (start 120.73 90.98) (end 120 90.98) (width 0.5) (layer "F.Cu") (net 2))
 (segment (start 112.8 86.35) (end 110.4 88.75) (width 0.5) (layer "F.Cu") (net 2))
 (segment (start 117.975 85.975) (end 119.4 87.4) (width 0.5) (layer "F.Cu") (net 2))
 (segment (start 118.475 88.325) (end 119.4 87.4) (width 0.2) (layer "F.Cu") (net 2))
 (segment (start 119.4 87.4) (end 121.1 89.1) (width 0.5) (layer "F.Cu") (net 2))
 (segment (start 115.15 97.3) (end 115.2 97.35) (width 0.5) (layer "F.Cu") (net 2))
 (segment (start 121.1 92.85) (end 123.75 95.5) (width 0.5) (layer "F.Cu") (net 2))
 (segment (start 115.525 86.35) (end 115.9 85.975) (width 0.5) (layer "F.Cu") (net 2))
 (segment (start 119.259999 92) (end 120 91.259999) (width 0.2) (layer "F.Cu") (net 2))
 (segment (start 110.4 88.75) (end 110.4 97.631371) (width 0.5) (layer "F.Cu") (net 2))
 (segment (start 117.5 85.975) (end 117.975 85.975) (width 0.5) (layer "F.Cu") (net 2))
 (segment (start 121.1 91) (end 120.75 91) (width 0.5) (layer "F.Cu") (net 2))
 (segment (start 114.15 98.4) (end 115.2 97.35) (width 0.5) (layer "F.Cu") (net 2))
 (segment (start 117.05 89) (end 117.725 88.325) (width 0.2) (layer "F.Cu") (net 2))
 (segment (start 115.9 85.975) (end 117.5 85.975) (width 0.5) (layer "F.Cu") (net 2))
 (segment (start 112.8 86.35) (end 115.525 86.35) (width 0.5) (layer "F.Cu") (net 2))
 (segment (start 113.23 97.3) (end 115.15 97.3) (width 0.5) (layer "F.Cu") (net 2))
 (segment (start 117.45 93.35) (end 117.45 92.5) (width 0.2) (layer "F.Cu") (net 5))
 (segment (start 118.5 94.4) (end 117.45 93.35) (width 0.2) (layer "F.Cu") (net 5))
 (segment (start 115.9 87.625) (end 115.825 87.625) (width 0.2) (layer "F.Cu") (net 3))
 (segment (start 116.25 87.975) (end 115.9 87.625) (width 0.2) (layer "F.Cu") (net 3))
 (segment (start 115.825 87.625) (end 114.56 88.89) (width 0.2) (layer "F.Cu") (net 3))
 (segment (start 114.56 88.89) (end 112.8 88.89) (width 0.2) (layer "F.Cu") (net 3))
 (segment (start 116.25 89.5) (end 116.25 87.975) (width 0.2) (layer "F.Cu") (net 3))
 (segment (start 111.65 88.413654) (end 111.65 90.28) (width 0.2) (layer "F.Cu") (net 7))
 (segment (start 112.538654 87.525) (end 114.812352 87.525) (width 0.2) (layer "F.Cu") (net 7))
 (segment (start 115.437352 86.9) (end 116.775 86.9) (width 0.2) (layer "F.Cu") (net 7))
 (segment (start 114.812352 87.525) (end 115.437352 86.9) (width 0.2) (layer "F.Cu") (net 7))
 (segment (start 116.65 88.75) (end 116.65 89.5) (width 0.2) (layer "F.Cu") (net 7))
 (segment (start 117.5 87.9) (end 116.65 88.75) (width 0.2) (layer "F.Cu") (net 7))
 (segment (start 116.775 86.9) (end 117.5 87.625) (width 0.2) (layer "F.Cu") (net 7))
 (segment (start 111.65 90.28) (end 112.8 91.43) (width 0.2) (layer "F.Cu") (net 7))
 (segment (start 112.538654 87.525) (end 111.65 88.413654) (width 0.2) (layer "F.Cu") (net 7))
 (segment (start 117.5 87.625) (end 117.5 87.9) (width 0.2) (layer "F.Cu") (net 7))
 (segment (start 123.62 92.63) (end 123.75 92.5) (width 0.2) (layer "F.Cu") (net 4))
 (segment (start 125.168629 97.631371) (end 125.168629 96.212742) (width 0.2) (layer "F.Cu") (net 4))
 (segment (start 123.45 97.7) (end 125.1 97.7) (width 0.2) (layer "F.Cu") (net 4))
 (segment (start 126.3 94.418629) (end 124.381371 92.5) (width 0.2) (layer "F.Cu") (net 4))
 (segment (start 124.381371 92.5) (end 123.75 92.5) (width 0.2) (layer "F.Cu") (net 4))
 (segment (start 126.3 95.081371) (end 126.3 94.418629) (width 0.2) (layer "F.Cu") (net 4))
 (segment (start 118.25 92.5) (end 123.45 97.7) (width 0.2) (layer "F.Cu") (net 4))
 (segment (start 125.1 97.7) (end 125.168629 97.631371) (width 0.2) (layer "F.Cu") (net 4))
 (segment (start 125.168629 96.212742) (end 126.3 95.081371) (width 0.2) (layer "F.Cu") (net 4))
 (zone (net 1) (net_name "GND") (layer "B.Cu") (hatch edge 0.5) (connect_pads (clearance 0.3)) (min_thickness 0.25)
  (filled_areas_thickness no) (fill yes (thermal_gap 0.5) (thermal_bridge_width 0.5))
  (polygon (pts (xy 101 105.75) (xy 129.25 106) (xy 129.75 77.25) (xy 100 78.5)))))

